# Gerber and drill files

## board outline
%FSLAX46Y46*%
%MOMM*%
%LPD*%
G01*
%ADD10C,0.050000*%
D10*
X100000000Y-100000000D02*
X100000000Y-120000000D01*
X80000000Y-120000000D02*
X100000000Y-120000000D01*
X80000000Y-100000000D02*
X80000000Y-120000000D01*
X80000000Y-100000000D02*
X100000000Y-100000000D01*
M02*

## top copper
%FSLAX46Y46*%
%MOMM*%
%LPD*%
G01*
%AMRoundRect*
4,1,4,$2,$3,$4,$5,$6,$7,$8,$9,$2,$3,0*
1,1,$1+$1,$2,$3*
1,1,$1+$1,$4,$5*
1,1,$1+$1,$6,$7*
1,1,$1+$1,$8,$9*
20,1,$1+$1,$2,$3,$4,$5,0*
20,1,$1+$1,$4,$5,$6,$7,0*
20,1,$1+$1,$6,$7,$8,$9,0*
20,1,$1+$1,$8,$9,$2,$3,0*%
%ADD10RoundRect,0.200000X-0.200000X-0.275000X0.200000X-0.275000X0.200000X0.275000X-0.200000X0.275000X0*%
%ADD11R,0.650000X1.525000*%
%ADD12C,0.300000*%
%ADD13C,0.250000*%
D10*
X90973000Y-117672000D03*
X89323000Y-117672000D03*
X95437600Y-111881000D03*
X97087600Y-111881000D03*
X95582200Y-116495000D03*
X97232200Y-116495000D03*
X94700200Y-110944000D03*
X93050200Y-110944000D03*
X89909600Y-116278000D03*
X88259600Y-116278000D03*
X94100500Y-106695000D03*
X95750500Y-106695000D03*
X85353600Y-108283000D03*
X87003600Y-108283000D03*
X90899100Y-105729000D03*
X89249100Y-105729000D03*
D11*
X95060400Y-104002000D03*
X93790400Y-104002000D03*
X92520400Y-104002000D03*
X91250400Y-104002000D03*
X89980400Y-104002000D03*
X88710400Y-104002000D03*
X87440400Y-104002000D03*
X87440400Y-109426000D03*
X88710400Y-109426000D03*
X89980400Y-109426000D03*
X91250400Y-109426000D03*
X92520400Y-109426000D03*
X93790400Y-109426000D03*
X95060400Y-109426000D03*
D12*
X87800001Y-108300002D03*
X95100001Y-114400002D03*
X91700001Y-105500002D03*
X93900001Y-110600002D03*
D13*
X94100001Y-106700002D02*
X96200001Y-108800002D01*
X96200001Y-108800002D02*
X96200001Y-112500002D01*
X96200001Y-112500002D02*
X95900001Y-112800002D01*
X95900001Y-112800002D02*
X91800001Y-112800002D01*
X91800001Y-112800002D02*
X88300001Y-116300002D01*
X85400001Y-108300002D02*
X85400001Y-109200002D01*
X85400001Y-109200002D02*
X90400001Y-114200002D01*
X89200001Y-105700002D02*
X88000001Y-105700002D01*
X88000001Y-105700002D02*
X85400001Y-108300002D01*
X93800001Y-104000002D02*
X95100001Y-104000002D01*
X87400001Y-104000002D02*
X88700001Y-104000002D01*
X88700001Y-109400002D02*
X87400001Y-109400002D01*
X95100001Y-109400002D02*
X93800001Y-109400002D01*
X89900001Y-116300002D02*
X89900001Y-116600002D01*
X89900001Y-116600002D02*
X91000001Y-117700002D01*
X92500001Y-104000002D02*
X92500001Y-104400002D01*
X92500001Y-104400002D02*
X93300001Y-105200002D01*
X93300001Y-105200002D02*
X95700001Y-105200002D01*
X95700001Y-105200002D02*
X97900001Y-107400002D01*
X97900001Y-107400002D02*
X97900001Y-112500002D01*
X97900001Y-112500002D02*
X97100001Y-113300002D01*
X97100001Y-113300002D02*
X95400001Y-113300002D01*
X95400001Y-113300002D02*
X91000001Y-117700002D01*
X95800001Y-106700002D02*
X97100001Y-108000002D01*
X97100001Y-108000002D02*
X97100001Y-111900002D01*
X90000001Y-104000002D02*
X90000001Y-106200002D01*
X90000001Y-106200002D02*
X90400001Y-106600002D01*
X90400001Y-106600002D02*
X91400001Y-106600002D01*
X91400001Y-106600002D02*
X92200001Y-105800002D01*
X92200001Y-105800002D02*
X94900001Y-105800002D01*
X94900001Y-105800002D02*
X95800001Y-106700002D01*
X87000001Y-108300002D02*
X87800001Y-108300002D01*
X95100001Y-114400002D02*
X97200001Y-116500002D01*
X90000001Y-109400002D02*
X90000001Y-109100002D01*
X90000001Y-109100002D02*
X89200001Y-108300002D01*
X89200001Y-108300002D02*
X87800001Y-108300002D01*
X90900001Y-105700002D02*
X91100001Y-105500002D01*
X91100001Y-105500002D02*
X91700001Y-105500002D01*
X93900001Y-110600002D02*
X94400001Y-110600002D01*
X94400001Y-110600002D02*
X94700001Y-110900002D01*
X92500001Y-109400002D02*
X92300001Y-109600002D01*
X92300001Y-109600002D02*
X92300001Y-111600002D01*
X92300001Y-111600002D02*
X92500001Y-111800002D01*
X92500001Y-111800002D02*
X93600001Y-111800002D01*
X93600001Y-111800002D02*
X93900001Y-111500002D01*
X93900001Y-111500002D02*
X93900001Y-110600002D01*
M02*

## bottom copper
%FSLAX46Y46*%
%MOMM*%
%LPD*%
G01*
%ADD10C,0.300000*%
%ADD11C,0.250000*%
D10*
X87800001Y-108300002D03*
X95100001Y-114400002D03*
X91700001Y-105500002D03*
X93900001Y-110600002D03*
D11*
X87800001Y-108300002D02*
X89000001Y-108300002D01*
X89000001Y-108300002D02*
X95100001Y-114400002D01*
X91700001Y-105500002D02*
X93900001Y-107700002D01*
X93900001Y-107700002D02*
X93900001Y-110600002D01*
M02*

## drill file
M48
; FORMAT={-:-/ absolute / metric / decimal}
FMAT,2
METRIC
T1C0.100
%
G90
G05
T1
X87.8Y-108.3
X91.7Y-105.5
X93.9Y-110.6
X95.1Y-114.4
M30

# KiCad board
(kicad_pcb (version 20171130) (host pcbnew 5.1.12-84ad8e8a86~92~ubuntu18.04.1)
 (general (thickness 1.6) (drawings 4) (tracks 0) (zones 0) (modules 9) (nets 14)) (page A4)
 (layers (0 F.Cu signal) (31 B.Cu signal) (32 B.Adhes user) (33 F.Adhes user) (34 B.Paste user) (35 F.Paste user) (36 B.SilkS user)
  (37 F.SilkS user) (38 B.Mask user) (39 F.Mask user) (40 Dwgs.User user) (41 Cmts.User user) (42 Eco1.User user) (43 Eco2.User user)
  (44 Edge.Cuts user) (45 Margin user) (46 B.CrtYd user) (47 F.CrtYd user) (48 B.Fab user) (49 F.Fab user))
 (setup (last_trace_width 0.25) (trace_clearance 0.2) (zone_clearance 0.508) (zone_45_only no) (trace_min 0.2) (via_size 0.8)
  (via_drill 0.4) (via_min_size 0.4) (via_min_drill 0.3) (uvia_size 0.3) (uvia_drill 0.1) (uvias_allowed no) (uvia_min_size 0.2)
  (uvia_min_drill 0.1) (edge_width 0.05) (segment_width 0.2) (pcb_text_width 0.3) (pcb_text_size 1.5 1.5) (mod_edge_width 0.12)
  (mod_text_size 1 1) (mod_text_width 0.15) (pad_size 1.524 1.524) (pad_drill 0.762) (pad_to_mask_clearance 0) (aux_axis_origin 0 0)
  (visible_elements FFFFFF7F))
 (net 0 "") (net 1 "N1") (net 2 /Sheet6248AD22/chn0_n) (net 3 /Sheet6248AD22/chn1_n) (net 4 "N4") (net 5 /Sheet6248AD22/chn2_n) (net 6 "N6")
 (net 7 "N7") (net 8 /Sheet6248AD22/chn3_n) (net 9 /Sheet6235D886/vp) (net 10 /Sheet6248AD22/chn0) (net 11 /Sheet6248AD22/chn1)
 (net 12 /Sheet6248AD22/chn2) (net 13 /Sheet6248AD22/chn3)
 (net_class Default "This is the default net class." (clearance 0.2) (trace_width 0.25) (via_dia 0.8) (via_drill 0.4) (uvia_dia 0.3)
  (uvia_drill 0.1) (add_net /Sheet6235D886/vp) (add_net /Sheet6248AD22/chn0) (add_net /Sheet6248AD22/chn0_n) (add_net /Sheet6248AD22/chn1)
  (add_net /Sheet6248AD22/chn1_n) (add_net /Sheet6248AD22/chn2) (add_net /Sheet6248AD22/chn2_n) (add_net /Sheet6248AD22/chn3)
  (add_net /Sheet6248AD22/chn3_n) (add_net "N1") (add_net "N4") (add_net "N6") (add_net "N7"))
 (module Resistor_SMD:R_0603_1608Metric (layer F.Cu) (at 90.148000 117.672000)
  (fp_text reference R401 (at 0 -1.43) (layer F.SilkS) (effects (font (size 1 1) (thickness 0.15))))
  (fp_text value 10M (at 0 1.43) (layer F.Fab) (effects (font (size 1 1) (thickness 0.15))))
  (pad 2 smd roundrect (at 0.825 0) (size 0.8 0.95) (layers F.Cu F.Mask F.Paste) (roundrect_rratio 0.25) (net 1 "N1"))
  (pad 1 smd roundrect (at -0.825 0) (size 0.8 0.95) (layers F.Cu F.Mask F.Paste) (roundrect_rratio 0.25) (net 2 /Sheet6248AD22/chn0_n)))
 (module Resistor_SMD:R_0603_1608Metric (layer F.Cu) (at 96.262600 111.881000)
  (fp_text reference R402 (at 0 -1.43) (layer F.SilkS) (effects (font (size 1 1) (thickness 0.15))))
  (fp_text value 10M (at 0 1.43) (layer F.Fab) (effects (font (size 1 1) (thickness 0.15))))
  (pad 1 smd roundrect (at -0.825 0) (size 0.8 0.95) (layers F.Cu F.Mask F.Paste) (roundrect_rratio 0.25) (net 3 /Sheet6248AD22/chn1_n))
  (pad 2 smd roundrect (at 0.825 0) (size 0.8 0.95) (layers F.Cu F.Mask F.Paste) (roundrect_rratio 0.25) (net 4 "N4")))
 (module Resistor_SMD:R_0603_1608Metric (layer F.Cu) (at 96.407200 116.495000)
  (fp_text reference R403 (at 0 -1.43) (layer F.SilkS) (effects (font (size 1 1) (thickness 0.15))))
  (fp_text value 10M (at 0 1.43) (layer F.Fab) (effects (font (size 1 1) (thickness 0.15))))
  (pad 1 smd roundrect (at -0.825 0) (size 0.8 0.95) (layers F.Cu F.Mask F.Paste) (roundrect_rratio 0.25) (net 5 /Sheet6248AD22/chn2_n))
  (pad 2 smd roundrect (at 0.825 0) (size 0.8 0.95) (layers F.Cu F.Mask F.Paste) (roundrect_rratio 0.25) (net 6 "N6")))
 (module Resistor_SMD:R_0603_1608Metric (layer F.Cu) (at 93.875200 110.944000)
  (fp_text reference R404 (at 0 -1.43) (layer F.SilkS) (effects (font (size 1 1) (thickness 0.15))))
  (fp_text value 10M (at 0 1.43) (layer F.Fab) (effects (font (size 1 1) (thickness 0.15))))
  (pad 2 smd roundrect (at 0.825 0) (size 0.8 0.95) (layers F.Cu F.Mask F.Paste) (roundrect_rratio 0.25) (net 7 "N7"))
  (pad 1 smd roundrect (at -0.825 0) (size 0.8 0.95) (layers F.Cu F.Mask F.Paste) (roundrect_rratio 0.25) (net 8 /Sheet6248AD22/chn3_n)))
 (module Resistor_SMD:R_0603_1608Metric (layer F.Cu) (at 89.084600 116.278000)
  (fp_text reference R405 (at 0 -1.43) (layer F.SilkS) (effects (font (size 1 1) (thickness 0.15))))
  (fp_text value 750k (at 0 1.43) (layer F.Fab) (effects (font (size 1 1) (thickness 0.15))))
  (pad 2 smd roundrect (at 0.825 0) (size 0.8 0.95) (layers F.Cu F.Mask F.Paste) (roundrect_rratio 0.25) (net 1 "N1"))
  (pad 1 smd roundrect (at -0.825 0) (size 0.8 0.95) (layers F.Cu F.Mask F.Paste) (roundrect_rratio 0.25) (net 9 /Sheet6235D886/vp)))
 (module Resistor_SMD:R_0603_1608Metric (layer F.Cu) (at 94.925500 106.695000)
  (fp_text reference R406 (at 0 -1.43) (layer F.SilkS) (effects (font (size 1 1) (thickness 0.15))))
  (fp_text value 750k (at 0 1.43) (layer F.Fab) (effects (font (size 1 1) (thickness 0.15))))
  (pad 1 smd roundrect (at -0.825 0) (size 0.8 0.95) (layers F.Cu F.Mask F.Paste) (roundrect_rratio 0.25) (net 9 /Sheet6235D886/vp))
  (pad 2 smd roundrect (at 0.825 0) (size 0.8 0.95) (layers F.Cu F.Mask F.Paste) (roundrect_rratio 0.25) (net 4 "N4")))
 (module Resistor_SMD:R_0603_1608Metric (layer F.Cu) (at 86.178600 108.283000)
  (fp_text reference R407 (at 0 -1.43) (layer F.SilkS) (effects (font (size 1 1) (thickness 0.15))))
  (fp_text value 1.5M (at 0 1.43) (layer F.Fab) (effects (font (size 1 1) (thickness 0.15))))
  (pad 1 smd roundrect (at -0.825 0) (size 0.8 0.95) (layers F.Cu F.Mask F.Paste) (roundrect_rratio 0.25) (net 9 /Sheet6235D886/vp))
  (pad 2 smd roundrect (at 0.825 0) (size 0.8 0.95) (layers F.Cu F.Mask F.Paste) (roundrect_rratio 0.25) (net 6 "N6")))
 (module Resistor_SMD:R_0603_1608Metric (layer F.Cu) (at 90.074100 105.729000)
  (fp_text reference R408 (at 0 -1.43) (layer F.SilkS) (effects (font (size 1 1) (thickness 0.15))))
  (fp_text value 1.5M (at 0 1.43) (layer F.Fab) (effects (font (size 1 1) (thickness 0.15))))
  (pad 2 smd roundrect (at 0.825 0) (size 0.8 0.95) (layers F.Cu F.Mask F.Paste) (roundrect_rratio 0.25) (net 7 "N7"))
  (pad 1 smd roundrect (at -0.825 0) (size 0.8 0.95) (layers F.Cu F.Mask F.Paste) (roundrect_rratio 0.25) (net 9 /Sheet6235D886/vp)))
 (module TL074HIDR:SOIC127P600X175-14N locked (layer F.Cu) (at 91.250400 106.714000 270.000000)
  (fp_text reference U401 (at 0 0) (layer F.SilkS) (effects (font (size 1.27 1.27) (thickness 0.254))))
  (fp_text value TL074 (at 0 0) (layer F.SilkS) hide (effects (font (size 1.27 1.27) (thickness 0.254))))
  (pad 1 smd rect (at -2.712 -3.81) (size 0.65 1.525) (layers F.Cu F.Mask F.Paste) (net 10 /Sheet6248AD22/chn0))
  (pad 2 smd rect (at -2.712 -2.54) (size 0.65 1.525) (layers F.Cu F.Mask F.Paste) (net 10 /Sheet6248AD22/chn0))
  (pad 3 smd rect (at -2.712 -1.27) (size 0.65 1.525) (layers F.Cu F.Mask F.Paste) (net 1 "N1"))
  (pad 4 smd rect (at -2.712 0) (size 0.65 1.525) (layers F.Cu F.Mask F.Paste))
  (pad 5 smd rect (at -2.712 1.27) (size 0.65 1.525) (layers F.Cu F.Mask F.Paste) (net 4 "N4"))
  (pad 6 smd rect (at -2.712 2.54) (size 0.65 1.525) (layers F.Cu F.Mask F.Paste) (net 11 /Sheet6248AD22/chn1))
  (pad 7 smd rect (at -2.712 3.81) (size 0.65 1.525) (layers F.Cu F.Mask F.Paste) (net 11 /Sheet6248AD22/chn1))
  (pad 8 smd rect (at 2.712 3.81) (size 0.65 1.525) (layers F.Cu F.Mask F.Paste) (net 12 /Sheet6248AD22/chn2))
  (pad 9 smd rect (at 2.712 2.54) (size 0.65 1.525) (layers F.Cu F.Mask F.Paste) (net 12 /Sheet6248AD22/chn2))
  (pad 10 smd rect (at 2.712 1.27) (size 0.65 1.525) (layers F.Cu F.Mask F.Paste) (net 6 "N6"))
  (pad 11 smd rect (at 2.712 0) (size 0.65 1.525) (layers F.Cu F.Mask F.Paste))
  (pad 12 smd rect (at 2.712 -1.27) (size 0.65 1.525) (layers F.Cu F.Mask F.Paste) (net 7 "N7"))
  (pad 13 smd rect (at 2.712 -2.54) (size 0.65 1.525) (layers F.Cu F.Mask F.Paste) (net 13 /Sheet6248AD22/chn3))
  (pad 14 smd rect (at 2.712 -3.81) (size 0.65 1.525) (layers F.Cu F.Mask F.Paste) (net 13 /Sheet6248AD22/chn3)))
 (gr_line (start 100 100) (end 100 120) (layer Edge.Cuts) (width 0.05))
 (gr_line (start 80 120) (end 100 120) (layer Edge.Cuts) (width 0.05))
 (gr_line (start 80 100) (end 80 120) (layer Edge.Cuts) (width 0.05))
 (gr_line (start 80 100) (end 100 100) (layer Edge.Cuts) (width 0.05))
 (segment (start 94.100001 106.700002) (end 96.200001 108.800002) (width 0.250000) (layer F.Cu) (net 9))
 (segment (start 96.200001 108.800002) (end 96.200001 112.500002) (width 0.250000) (layer F.Cu) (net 9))
 (segment (start 96.200001 112.500002) (end 95.900001 112.800002) (width 0.250000) (layer F.Cu) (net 9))
 (segment (start 95.900001 112.800002) (end 91.800001 112.800002) (width 0.250000) (layer F.Cu) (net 9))
 (segment (start 91.800001 112.800002) (end 88.300001 116.300002) (width 0.250000) (layer F.Cu) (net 9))
 (segment (start 85.400001 108.300002) (end 85.400001 109.200002) (width 0.250000) (layer F.Cu) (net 9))
 (segment (start 85.400001 109.200002) (end 90.400001 114.200002) (width 0.250000) (layer F.Cu) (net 9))
 (segment (start 89.200001 105.700002) (end 88.000001 105.700002) (width 0.250000) (layer F.Cu) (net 9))
 (segment (start 88.000001 105.700002) (end 85.400001 108.300002) (width 0.250000) (layer F.Cu) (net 9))
 (segment (start 93.800001 104.000002) (end 95.100001 104.000002) (width 0.250000) (layer F.Cu) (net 10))
 (segment (start 87.400001 104.000002) (end 88.700001 104.000002) (width 0.250000) (layer F.Cu) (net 11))
 (segment (start 88.700001 109.400002) (end 87.400001 109.400002) (width 0.250000) (layer F.Cu) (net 12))
 (segment (start 95.100001 109.400002) (end 93.800001 109.400002) (width 0.250000) (layer F.Cu) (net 13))
 (segment (start 89.900001 116.300002) (end 89.900001 116.600002) (width 0.250000) (layer F.Cu) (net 1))
 (segment (start 89.900001 116.600002) (end 91.000001 117.700002) (width 0.250000) (layer F.Cu) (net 1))
 (segment (start 92.500001 104.000002) (end 92.500001 104.400002) (width 0.250000) (layer F.Cu) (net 1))
 (segment (start 92.500001 104.400002) (end 93.300001 105.200002) (width 0.250000) (layer F.Cu) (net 1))
 (segment (start 93.300001 105.200002) (end 95.700001 105.200002) (width 0.250000) (layer F.Cu) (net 1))
 (segment (start 95.700001 105.200002) (end 97.900001 107.400002) (width 0.250000) (layer F.Cu) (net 1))
 (segment (start 97.900001 107.400002) (end 97.900001 112.500002) (width 0.250000) (layer F.Cu) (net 1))
 (segment (start 97.900001 112.500002) (end 97.100001 113.300002) (width 0.250000) (layer F.Cu) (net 1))
 (segment (start 97.100001 113.300002) (end 95.400001 113.300002) (width 0.250000) (layer F.Cu) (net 1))
 (segment (start 95.400001 113.300002) (end 91.000001 117.700002) (width 0.250000) (layer F.Cu) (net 1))
 (segment (start 95.800001 106.700002) (end 97.100001 108.000002) (width 0.250000) (layer F.Cu) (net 4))
 (segment (start 97.100001 108.000002) (end 97.100001 111.900002) (width 0.250000) (layer F.Cu) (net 4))
 (segment (start 90.000001 104.000002) (end 90.000001 106.200002) (width 0.250000) (layer F.Cu) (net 4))
 (segment (start 90.000001 106.200002) (end 90.400001 106.600002) (width 0.250000) (layer F.Cu) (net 4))
 (segment (start 90.400001 106.600002) (end 91.400001 106.600002) (width 0.250000) (layer F.Cu) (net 4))
 (segment (start 91.400001 106.600002) (end 92.200001 105.800002) (width 0.250000) (layer F.Cu) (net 4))
 (segment (start 92.200001 105.800002) (end 94.900001 105.800002) (width 0.250000) (layer F.Cu) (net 4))
 (segment (start 94.900001 105.800002) (end 95.800001 106.700002) (width 0.250000) (layer F.Cu) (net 4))
 (segment (start 87.000001 108.300002) (end 87.800001 108.300002) (width 0.250000) (layer F.Cu) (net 6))
 (segment (start 87.800001 108.300002) (end 89.000001 108.300002) (width 0.250000) (layer B.Cu) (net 6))
 (segment (start 89.000001 108.300002) (end 95.100001 114.400002) (width 0.250000) (layer B.Cu) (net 6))
 (segment (start 95.100001 114.400002) (end 97.200001 116.500002) (width 0.250000) (layer F.Cu) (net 6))
 (segment (start 90.000001 109.400002) (end 90.000001 109.100002) (width 0.250000) (layer F.Cu) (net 6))
 (segment (start 90.000001 109.100002) (end 89.200001 108.300002) (width 0.250000) (layer F.Cu) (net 6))
 (segment (start 89.200001 108.300002) (end 87.800001 108.300002) (width 0.250000) (layer F.Cu) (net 6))
 (via micro (at 87.800001 108.300002) (size 0.300000) (drill 0.100000) (layers F.Cu B.Cu) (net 6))
 (via micro (at 95.100001 114.400002) (size 0.300000) (drill 0.100000) (layers F.Cu B.Cu) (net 6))
 (segment (start 90.900001 105.700002) (end 91.100001 105.500002) (width 0.250000) (layer F.Cu) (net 7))
 (segment (start 91.100001 105.500002) (end 91.700001 105.500002) (width 0.250000) (layer F.Cu) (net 7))
 (segment (start 91.700001 105.500002) (end 93.900001 107.700002) (width 0.250000) (layer B.Cu) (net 7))
 (segment (start 93.900001 107.700002) (end 93.900001 110.600002) (width 0.250000) (layer B.Cu) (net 7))
 (segment (start 93.900001 110.600002) (end 94.400001 110.600002) (width 0.250000) (layer F.Cu) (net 7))
 (segment (start 94.400001 110.600002) (end 94.700001 110.900002) (width 0.250000) (layer F.Cu) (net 7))
 (segment (start 92.500001 109.400002) (end 92.300001 109.600002) (width 0.250000) (layer F.Cu) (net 7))
 (segment (start 92.300001 109.600002) (end 92.300001 111.600002) (width 0.250000) (layer F.Cu) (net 7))
 (segment (start 92.300001 111.600002) (end 92.500001 111.800002) (width 0.250000) (layer F.Cu) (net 7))
 (segment (start 92.500001 111.800002) (end 93.600001 111.800002) (width 0.250000) (layer F.Cu) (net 7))
 (segment (start 93.600001 111.800002) (end 93.900001 111.500002) (width 0.250000) (layer F.Cu) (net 7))
 (segment (start 93.900001 111.500002) (end 93.900001 110.600002) (width 0.250000) (layer F.Cu) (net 7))
 (via micro (at 91.700001 105.500002) (size 0.300000) (drill 0.100000) (layers F.Cu B.Cu) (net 7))
 (via micro (at 93.900001 110.600002) (size 0.300000) (drill 0.100000) (layers F.Cu B.Cu) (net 7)))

